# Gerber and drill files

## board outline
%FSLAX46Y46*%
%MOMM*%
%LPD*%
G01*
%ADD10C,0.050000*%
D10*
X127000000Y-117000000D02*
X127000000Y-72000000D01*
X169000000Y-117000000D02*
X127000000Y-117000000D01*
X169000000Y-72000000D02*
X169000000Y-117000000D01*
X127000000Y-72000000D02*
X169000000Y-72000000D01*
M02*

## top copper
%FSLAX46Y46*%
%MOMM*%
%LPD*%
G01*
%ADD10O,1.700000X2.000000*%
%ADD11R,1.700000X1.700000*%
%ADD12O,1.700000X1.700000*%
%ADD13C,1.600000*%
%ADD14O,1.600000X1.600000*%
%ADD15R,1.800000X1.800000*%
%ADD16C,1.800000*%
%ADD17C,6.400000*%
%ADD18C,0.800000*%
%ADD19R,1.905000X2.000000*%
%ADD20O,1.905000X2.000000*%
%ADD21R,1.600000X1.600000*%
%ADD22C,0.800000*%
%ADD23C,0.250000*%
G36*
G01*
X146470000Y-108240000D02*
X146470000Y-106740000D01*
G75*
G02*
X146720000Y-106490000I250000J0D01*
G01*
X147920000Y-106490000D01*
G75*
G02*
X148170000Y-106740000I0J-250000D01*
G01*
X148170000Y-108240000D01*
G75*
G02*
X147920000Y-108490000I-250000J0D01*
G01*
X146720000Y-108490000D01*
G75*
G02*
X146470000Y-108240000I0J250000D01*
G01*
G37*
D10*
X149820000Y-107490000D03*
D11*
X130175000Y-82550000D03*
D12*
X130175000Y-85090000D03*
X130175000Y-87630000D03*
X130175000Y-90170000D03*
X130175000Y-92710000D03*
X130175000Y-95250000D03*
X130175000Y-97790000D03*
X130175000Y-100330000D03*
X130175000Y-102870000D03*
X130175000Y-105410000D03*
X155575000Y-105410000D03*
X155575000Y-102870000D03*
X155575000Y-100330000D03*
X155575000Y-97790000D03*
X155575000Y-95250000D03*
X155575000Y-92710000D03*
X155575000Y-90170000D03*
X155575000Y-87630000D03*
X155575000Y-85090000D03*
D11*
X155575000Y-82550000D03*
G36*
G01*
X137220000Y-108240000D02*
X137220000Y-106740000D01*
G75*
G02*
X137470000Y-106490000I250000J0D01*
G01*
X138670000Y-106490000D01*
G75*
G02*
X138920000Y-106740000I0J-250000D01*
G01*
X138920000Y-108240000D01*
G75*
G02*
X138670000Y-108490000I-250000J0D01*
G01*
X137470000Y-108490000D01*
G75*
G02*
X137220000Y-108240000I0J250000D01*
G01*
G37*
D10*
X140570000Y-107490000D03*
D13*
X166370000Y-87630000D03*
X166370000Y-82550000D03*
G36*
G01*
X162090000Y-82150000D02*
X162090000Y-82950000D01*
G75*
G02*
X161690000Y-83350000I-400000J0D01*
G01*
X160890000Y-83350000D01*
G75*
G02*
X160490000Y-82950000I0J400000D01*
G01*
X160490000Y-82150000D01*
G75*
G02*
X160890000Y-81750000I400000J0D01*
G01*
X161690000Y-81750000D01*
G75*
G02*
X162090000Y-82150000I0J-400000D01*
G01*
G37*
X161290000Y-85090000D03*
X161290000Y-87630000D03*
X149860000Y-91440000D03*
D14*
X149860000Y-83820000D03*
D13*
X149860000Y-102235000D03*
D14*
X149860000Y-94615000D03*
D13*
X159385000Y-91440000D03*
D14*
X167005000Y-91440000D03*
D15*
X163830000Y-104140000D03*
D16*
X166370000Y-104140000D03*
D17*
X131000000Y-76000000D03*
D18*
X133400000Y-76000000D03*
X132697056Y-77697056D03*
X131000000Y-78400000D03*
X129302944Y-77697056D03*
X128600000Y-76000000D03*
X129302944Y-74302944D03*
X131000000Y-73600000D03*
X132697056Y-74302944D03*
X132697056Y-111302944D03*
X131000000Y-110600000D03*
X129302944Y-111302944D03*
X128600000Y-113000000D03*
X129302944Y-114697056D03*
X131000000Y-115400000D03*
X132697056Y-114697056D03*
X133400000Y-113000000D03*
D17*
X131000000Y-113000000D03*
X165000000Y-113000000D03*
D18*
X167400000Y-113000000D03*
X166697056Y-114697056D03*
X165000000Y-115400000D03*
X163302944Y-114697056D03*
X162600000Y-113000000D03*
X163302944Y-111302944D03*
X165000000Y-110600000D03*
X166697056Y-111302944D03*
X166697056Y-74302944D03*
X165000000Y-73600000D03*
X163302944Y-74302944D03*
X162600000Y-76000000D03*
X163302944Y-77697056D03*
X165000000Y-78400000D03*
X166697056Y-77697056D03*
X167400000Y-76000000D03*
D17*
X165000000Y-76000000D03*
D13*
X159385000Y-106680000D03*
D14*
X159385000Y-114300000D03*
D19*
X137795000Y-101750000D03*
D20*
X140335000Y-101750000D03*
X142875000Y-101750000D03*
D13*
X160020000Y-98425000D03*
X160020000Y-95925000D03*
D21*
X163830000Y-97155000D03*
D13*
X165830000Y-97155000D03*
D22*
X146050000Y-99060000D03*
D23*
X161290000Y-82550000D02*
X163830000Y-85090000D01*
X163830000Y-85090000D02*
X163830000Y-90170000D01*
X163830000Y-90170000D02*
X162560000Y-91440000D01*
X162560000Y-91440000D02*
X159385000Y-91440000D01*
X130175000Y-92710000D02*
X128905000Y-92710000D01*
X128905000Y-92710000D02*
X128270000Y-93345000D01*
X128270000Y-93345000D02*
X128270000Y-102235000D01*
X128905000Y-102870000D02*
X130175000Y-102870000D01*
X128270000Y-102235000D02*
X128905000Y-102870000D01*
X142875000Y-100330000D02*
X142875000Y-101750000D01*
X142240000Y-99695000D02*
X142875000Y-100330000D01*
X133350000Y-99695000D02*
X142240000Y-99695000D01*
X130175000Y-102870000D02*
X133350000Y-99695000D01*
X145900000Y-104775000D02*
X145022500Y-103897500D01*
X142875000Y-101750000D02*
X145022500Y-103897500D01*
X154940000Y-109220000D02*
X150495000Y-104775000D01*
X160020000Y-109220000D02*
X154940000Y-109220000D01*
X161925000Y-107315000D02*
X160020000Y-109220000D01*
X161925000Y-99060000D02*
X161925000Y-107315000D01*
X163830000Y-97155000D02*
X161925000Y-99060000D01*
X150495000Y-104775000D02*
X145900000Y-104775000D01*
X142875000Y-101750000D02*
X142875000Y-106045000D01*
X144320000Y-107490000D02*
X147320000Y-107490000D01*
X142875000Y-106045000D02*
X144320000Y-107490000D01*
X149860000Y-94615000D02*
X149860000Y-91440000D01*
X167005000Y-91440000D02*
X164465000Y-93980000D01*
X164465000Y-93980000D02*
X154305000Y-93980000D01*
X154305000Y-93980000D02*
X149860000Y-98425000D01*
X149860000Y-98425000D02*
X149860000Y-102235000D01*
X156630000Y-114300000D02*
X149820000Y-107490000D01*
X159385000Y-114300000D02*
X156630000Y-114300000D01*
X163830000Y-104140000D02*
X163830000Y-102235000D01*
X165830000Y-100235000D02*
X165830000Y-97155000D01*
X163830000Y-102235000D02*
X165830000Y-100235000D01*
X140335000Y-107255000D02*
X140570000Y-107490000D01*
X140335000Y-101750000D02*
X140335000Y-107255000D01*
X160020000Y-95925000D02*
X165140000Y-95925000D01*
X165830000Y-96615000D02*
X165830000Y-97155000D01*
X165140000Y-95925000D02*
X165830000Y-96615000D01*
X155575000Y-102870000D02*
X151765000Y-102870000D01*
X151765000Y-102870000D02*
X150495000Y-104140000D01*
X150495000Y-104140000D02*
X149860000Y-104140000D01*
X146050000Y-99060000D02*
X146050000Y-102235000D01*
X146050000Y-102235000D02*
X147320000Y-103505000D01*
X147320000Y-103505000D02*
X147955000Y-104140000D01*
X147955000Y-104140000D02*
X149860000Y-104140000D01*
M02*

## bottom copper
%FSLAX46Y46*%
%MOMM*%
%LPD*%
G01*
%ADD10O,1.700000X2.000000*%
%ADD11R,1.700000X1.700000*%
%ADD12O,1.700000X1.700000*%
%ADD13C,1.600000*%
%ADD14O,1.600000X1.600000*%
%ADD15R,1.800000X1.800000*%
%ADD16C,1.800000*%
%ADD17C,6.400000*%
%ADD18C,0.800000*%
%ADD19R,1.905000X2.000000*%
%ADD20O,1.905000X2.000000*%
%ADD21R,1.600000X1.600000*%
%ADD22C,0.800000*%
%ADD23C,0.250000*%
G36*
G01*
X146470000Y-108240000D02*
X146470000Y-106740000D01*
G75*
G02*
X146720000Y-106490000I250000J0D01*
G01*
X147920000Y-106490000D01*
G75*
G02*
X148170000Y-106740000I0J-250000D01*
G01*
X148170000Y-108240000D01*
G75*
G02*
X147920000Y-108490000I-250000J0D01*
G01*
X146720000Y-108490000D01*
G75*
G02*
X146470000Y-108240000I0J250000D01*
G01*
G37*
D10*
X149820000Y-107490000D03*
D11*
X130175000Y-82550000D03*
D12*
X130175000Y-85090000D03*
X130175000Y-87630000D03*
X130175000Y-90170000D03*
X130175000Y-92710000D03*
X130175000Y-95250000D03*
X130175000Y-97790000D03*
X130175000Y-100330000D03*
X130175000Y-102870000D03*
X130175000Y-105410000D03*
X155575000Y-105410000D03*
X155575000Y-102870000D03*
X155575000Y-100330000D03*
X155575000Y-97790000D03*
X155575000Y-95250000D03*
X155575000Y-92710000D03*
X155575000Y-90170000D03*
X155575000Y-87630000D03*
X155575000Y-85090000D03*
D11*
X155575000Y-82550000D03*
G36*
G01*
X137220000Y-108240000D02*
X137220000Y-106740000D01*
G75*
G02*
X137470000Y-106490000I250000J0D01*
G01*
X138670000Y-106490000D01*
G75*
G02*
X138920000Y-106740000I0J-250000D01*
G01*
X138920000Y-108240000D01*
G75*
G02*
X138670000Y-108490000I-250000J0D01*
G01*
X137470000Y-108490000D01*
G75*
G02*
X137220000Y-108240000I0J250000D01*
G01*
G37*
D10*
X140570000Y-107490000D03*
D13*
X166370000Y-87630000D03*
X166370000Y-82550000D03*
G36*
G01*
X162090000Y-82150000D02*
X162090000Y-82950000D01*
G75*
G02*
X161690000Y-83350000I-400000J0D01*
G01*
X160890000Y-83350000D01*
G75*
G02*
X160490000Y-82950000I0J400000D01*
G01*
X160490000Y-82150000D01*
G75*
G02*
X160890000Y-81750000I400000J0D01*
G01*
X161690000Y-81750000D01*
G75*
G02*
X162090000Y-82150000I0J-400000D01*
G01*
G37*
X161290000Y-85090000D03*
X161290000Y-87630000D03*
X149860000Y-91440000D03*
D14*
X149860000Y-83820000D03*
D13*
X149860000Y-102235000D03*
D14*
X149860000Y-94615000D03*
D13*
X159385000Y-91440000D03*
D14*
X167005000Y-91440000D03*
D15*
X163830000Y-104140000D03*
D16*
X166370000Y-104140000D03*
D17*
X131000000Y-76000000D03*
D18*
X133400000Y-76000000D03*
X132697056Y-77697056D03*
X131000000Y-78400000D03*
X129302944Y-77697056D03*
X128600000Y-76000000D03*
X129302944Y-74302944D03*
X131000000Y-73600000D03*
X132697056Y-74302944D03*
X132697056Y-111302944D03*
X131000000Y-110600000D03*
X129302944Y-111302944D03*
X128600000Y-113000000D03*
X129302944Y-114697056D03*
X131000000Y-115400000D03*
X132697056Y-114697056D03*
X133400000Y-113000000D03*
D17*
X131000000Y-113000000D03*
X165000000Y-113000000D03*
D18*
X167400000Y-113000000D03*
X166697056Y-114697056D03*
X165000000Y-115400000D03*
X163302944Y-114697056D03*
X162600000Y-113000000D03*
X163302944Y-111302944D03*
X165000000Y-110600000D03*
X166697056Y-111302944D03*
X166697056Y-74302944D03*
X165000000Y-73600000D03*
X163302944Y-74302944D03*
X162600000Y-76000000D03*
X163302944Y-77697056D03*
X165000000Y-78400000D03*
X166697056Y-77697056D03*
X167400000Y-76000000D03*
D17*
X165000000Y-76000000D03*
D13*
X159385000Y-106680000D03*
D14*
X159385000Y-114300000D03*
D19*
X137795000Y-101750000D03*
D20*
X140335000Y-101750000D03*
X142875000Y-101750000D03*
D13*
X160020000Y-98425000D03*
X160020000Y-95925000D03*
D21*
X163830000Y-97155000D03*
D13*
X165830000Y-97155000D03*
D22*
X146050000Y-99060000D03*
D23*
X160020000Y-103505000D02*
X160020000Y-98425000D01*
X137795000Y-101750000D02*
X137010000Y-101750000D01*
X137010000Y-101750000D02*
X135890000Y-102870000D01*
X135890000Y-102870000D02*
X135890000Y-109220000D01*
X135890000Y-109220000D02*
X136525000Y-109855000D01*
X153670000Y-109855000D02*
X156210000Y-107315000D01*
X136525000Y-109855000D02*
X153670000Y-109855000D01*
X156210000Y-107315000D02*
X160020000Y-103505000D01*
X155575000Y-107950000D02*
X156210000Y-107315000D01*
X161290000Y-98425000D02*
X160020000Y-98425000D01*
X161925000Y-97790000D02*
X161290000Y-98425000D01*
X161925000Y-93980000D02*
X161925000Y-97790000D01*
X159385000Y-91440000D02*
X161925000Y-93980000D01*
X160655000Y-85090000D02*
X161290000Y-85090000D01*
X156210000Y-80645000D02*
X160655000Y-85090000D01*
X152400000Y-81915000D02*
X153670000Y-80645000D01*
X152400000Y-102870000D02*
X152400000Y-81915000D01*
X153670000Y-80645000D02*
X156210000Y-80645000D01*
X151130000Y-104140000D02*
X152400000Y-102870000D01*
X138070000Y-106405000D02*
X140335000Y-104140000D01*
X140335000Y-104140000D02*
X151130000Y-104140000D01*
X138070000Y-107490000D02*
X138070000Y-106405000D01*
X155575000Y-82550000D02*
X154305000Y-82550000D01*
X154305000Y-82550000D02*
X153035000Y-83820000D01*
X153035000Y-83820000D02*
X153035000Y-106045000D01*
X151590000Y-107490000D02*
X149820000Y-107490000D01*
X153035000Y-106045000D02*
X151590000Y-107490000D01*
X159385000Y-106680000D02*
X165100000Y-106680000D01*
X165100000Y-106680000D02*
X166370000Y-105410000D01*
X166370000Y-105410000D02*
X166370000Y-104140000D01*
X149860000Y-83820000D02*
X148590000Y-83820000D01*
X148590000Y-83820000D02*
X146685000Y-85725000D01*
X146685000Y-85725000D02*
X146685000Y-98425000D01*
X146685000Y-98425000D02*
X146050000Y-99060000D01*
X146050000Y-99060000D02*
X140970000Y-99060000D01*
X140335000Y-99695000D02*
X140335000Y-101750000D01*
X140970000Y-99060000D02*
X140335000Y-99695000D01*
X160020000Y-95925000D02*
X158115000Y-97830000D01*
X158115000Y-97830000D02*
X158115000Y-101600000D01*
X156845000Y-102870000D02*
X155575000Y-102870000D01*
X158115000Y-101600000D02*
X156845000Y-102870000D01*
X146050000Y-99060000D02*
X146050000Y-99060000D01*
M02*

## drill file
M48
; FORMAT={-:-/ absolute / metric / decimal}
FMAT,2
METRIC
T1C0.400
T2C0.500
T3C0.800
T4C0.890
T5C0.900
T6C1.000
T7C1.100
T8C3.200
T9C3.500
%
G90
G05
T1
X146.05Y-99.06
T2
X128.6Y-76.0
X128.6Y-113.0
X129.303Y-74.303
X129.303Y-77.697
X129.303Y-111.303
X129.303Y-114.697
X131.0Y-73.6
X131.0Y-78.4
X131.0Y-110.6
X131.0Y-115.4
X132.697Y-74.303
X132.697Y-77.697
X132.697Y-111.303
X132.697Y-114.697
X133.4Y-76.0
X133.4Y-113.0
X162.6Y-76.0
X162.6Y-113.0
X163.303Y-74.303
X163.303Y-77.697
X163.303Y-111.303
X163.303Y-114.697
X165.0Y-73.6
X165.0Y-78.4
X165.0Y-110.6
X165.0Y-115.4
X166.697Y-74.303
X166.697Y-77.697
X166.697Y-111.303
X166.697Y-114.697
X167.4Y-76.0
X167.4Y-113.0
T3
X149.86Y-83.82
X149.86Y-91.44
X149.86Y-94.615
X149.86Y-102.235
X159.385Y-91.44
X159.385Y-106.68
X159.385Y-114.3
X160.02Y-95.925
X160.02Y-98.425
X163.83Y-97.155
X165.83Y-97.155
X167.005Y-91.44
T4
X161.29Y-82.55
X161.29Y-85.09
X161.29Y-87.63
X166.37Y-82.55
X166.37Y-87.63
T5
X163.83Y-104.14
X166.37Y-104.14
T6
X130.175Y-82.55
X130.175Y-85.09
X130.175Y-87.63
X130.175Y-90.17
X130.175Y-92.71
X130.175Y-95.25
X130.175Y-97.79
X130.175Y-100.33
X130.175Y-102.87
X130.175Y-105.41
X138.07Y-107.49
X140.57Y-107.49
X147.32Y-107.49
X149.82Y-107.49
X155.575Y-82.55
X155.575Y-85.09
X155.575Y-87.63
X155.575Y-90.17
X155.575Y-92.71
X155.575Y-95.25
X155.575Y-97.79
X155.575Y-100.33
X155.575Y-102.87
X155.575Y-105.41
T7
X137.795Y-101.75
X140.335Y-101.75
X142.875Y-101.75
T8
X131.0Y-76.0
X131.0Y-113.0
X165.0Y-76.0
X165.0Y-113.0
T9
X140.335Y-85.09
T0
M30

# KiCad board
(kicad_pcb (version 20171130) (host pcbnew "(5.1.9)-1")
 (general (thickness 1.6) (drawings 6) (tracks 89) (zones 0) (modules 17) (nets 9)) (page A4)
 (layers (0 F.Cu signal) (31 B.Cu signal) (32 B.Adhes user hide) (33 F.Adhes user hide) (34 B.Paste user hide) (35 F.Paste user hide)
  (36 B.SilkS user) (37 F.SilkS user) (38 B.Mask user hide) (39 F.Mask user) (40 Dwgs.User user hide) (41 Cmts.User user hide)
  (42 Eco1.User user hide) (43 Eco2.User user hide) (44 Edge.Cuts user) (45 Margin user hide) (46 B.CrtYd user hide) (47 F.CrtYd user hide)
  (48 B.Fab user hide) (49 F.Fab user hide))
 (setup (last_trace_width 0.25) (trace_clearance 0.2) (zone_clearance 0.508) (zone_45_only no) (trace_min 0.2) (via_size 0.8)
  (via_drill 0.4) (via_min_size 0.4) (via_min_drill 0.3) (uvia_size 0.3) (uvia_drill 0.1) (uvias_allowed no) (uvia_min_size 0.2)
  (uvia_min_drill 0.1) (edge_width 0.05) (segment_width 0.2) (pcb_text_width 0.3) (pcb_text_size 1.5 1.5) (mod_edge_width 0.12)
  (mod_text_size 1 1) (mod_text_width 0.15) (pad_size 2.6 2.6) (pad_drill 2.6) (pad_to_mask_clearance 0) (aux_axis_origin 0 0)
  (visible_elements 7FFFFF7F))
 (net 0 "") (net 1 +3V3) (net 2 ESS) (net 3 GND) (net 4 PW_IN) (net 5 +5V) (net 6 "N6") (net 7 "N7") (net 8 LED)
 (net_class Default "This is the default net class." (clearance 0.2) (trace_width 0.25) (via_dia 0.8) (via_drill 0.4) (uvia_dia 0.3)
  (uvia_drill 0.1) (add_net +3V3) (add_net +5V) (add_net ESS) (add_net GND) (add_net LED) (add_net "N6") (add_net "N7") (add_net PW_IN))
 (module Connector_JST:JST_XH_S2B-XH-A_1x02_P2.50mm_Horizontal (layer F.Cu) (at 147.32 107.49)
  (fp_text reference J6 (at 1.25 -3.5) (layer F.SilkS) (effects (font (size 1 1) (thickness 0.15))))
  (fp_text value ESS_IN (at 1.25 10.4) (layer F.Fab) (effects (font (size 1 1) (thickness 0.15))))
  (pad 1 thru_hole roundrect (at 0 0) (size 1.7 2) (drill 1) (layers *.Cu *.Mask) (roundrect_rratio 0.1470588235294118) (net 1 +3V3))
  (pad 2 thru_hole oval (at 2.5 0) (size 1.7 2) (drill 1) (layers *.Cu *.Mask) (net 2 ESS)))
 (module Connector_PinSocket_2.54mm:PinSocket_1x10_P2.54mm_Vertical (layer F.Cu) (at 130.175 82.55)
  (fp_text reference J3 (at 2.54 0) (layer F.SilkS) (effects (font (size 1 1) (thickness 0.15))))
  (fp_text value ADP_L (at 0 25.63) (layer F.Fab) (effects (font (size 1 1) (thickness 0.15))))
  (pad 1 thru_hole rect (at 0 0) (size 1.7 1.7) (drill 1) (layers *.Cu *.Mask))
  (pad 2 thru_hole oval (at 0 2.54) (size 1.7 1.7) (drill 1) (layers *.Cu *.Mask))
  (pad 3 thru_hole oval (at 0 5.08) (size 1.7 1.7) (drill 1) (layers *.Cu *.Mask))
  (pad 4 thru_hole oval (at 0 7.62) (size 1.7 1.7) (drill 1) (layers *.Cu *.Mask))
  (pad 5 thru_hole oval (at 0 10.16) (size 1.7 1.7) (drill 1) (layers *.Cu *.Mask) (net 1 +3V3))
  (pad 6 thru_hole oval (at 0 12.7) (size 1.7 1.7) (drill 1) (layers *.Cu *.Mask))
  (pad 7 thru_hole oval (at 0 15.24) (size 1.7 1.7) (drill 1) (layers *.Cu *.Mask))
  (pad 8 thru_hole oval (at 0 17.78) (size 1.7 1.7) (drill 1) (layers *.Cu *.Mask))
  (pad 9 thru_hole oval (at 0 20.32) (size 1.7 1.7) (drill 1) (layers *.Cu *.Mask) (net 1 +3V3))
  (pad 10 thru_hole oval (at 0 22.86) (size 1.7 1.7) (drill 1) (layers *.Cu *.Mask)))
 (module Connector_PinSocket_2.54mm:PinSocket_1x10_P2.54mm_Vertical (layer F.Cu) (at 155.575 82.55)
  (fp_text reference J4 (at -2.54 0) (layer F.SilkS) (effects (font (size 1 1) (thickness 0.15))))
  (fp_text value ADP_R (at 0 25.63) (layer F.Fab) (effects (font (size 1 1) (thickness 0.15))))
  (pad 10 thru_hole oval (at 0 22.86) (size 1.7 1.7) (drill 1) (layers *.Cu *.Mask))
  (pad 9 thru_hole oval (at 0 20.32) (size 1.7 1.7) (drill 1) (layers *.Cu *.Mask) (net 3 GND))
  (pad 8 thru_hole oval (at 0 17.78) (size 1.7 1.7) (drill 1) (layers *.Cu *.Mask))
  (pad 7 thru_hole oval (at 0 15.24) (size 1.7 1.7) (drill 1) (layers *.Cu *.Mask))
  (pad 6 thru_hole oval (at 0 12.7) (size 1.7 1.7) (drill 1) (layers *.Cu *.Mask))
  (pad 5 thru_hole oval (at 0 10.16) (size 1.7 1.7) (drill 1) (layers *.Cu *.Mask))
  (pad 4 thru_hole oval (at 0 7.62) (size 1.7 1.7) (drill 1) (layers *.Cu *.Mask))
  (pad 3 thru_hole oval (at 0 5.08) (size 1.7 1.7) (drill 1) (layers *.Cu *.Mask))
  (pad 2 thru_hole oval (at 0 2.54) (size 1.7 1.7) (drill 1) (layers *.Cu *.Mask))
  (pad 1 thru_hole rect (at 0 0) (size 1.7 1.7) (drill 1) (layers *.Cu *.Mask) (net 2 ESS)))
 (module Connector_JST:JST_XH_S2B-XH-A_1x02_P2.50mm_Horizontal (layer F.Cu) (at 138.07 107.49)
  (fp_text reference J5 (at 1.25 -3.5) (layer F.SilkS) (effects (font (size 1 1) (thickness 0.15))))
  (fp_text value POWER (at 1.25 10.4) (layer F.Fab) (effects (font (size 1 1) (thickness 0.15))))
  (pad 1 thru_hole roundrect (at 0 0) (size 1.7 2) (drill 1) (layers *.Cu *.Mask) (roundrect_rratio 0.1470588235294118) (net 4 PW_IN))
  (pad 2 thru_hole oval (at 2.5 0) (size 1.7 2) (drill 1) (layers *.Cu *.Mask) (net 3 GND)))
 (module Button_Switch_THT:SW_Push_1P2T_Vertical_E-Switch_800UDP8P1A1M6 (layer F.Cu) (at 161.29 82.55)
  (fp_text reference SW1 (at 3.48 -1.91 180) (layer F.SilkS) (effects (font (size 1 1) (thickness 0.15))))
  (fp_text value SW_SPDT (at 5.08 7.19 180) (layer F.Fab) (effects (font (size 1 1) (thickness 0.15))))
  (pad "" thru_hole circle (at 5.08 5.08 180) (size 1.6 1.6) (drill 0.89) (layers *.Cu *.Mask))
  (pad "" thru_hole circle (at 5.08 0 180) (size 1.6 1.6) (drill 0.89) (layers *.Cu *.Mask))
  (pad 1 thru_hole roundrect (at 0 0 180) (size 1.6 1.6) (drill 0.89) (layers *.Cu *.Mask) (roundrect_rratio 0.25) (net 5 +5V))
  (pad 2 thru_hole circle (at 0 2.54 180) (size 1.6 1.6) (drill 0.89) (layers *.Cu *.Mask) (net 4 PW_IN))
  (pad 3 thru_hole circle (at 0 5.08 180) (size 1.6 1.6) (drill 0.89) (layers *.Cu *.Mask)))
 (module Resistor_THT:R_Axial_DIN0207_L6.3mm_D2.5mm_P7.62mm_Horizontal (layer F.Cu) (at 149.86 91.44 90)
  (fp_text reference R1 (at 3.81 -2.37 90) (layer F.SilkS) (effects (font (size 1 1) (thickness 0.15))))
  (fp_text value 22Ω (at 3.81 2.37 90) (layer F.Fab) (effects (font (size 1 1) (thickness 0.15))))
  (pad 1 thru_hole circle (at 0 0 90) (size 1.6 1.6) (drill 0.8) (layers *.Cu *.Mask) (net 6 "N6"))
  (pad 2 thru_hole oval (at 7.62 0 90) (size 1.6 1.6) (drill 0.8) (layers *.Cu *.Mask) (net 3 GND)))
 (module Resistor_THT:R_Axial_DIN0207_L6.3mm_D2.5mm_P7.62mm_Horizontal (layer F.Cu) (at 149.86 102.235 90)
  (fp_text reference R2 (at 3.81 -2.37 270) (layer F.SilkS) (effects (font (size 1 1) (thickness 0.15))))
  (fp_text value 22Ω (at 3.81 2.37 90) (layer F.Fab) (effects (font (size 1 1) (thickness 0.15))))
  (pad 1 thru_hole circle (at 0 0 90) (size 1.6 1.6) (drill 0.8) (layers *.Cu *.Mask) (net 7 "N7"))
  (pad 2 thru_hole oval (at 7.62 0 90) (size 1.6 1.6) (drill 0.8) (layers *.Cu *.Mask) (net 6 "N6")))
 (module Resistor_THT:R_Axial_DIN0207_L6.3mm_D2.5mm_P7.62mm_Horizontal (layer F.Cu) (at 159.385 91.44)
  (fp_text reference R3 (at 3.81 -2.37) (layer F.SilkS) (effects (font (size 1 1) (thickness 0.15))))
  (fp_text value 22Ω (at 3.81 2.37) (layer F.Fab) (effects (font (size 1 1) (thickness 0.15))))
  (pad 1 thru_hole circle (at 0 0) (size 1.6 1.6) (drill 0.8) (layers *.Cu *.Mask) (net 5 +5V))
  (pad 2 thru_hole oval (at 7.62 0) (size 1.6 1.6) (drill 0.8) (layers *.Cu *.Mask) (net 7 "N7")))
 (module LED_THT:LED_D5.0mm (layer F.Cu) (at 163.83 104.14)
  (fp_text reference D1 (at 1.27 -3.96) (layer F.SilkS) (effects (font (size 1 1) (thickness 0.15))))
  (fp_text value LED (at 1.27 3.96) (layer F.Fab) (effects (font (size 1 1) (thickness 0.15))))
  (pad 1 thru_hole rect (at 0 0) (size 1.8 1.8) (drill 0.9) (layers *.Cu *.Mask) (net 3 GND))
  (pad 2 thru_hole circle (at 2.54 0) (size 1.8 1.8) (drill 0.9) (layers *.Cu *.Mask) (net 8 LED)))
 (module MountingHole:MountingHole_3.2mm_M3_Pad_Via (layer F.Cu) (at 131 76)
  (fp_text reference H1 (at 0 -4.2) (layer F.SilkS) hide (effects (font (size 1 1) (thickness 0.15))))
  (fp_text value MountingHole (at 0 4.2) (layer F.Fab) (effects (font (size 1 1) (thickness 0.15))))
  (pad 1 thru_hole circle (at 0 0) (size 6.4 6.4) (drill 3.2) (layers *.Cu *.Mask))
  (pad 1 thru_hole circle (at 2.4 0) (size 0.8 0.8) (drill 0.5) (layers *.Cu *.Mask))
  (pad 1 thru_hole circle (at 1.697056 1.697056) (size 0.8 0.8) (drill 0.5) (layers *.Cu *.Mask))
  (pad 1 thru_hole circle (at 0 2.4) (size 0.8 0.8) (drill 0.5) (layers *.Cu *.Mask))
  (pad 1 thru_hole circle (at -1.697056 1.697056) (size 0.8 0.8) (drill 0.5) (layers *.Cu *.Mask))
  (pad 1 thru_hole circle (at -2.4 0) (size 0.8 0.8) (drill 0.5) (layers *.Cu *.Mask))
  (pad 1 thru_hole circle (at -1.697056 -1.697056) (size 0.8 0.8) (drill 0.5) (layers *.Cu *.Mask))
  (pad 1 thru_hole circle (at 0 -2.4) (size 0.8 0.8) (drill 0.5) (layers *.Cu *.Mask))
  (pad 1 thru_hole circle (at 1.697056 -1.697056) (size 0.8 0.8) (drill 0.5) (layers *.Cu *.Mask)))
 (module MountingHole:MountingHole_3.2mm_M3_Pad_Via (layer F.Cu) (at 131 113)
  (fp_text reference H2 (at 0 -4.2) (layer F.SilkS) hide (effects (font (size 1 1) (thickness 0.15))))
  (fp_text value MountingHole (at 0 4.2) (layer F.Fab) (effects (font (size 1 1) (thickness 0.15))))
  (pad 1 thru_hole circle (at 1.697056 -1.697056) (size 0.8 0.8) (drill 0.5) (layers *.Cu *.Mask))
  (pad 1 thru_hole circle (at 0 -2.4) (size 0.8 0.8) (drill 0.5) (layers *.Cu *.Mask))
  (pad 1 thru_hole circle (at -1.697056 -1.697056) (size 0.8 0.8) (drill 0.5) (layers *.Cu *.Mask))
  (pad 1 thru_hole circle (at -2.4 0) (size 0.8 0.8) (drill 0.5) (layers *.Cu *.Mask))
  (pad 1 thru_hole circle (at -1.697056 1.697056) (size 0.8 0.8) (drill 0.5) (layers *.Cu *.Mask))
  (pad 1 thru_hole circle (at 0 2.4) (size 0.8 0.8) (drill 0.5) (layers *.Cu *.Mask))
  (pad 1 thru_hole circle (at 1.697056 1.697056) (size 0.8 0.8) (drill 0.5) (layers *.Cu *.Mask))
  (pad 1 thru_hole circle (at 2.4 0) (size 0.8 0.8) (drill 0.5) (layers *.Cu *.Mask))
  (pad 1 thru_hole circle (at 0 0) (size 6.4 6.4) (drill 3.2) (layers *.Cu *.Mask)))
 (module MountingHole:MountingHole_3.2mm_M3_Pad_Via (layer F.Cu) (at 165 113)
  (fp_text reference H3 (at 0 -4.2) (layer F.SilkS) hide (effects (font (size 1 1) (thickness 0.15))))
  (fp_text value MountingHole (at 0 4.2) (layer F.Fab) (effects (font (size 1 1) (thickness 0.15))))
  (pad 1 thru_hole circle (at 0 0) (size 6.4 6.4) (drill 3.2) (layers *.Cu *.Mask))
  (pad 1 thru_hole circle (at 2.4 0) (size 0.8 0.8) (drill 0.5) (layers *.Cu *.Mask))
  (pad 1 thru_hole circle (at 1.697056 1.697056) (size 0.8 0.8) (drill 0.5) (layers *.Cu *.Mask))
  (pad 1 thru_hole circle (at 0 2.4) (size 0.8 0.8) (drill 0.5) (layers *.Cu *.Mask))
  (pad 1 thru_hole circle (at -1.697056 1.697056) (size 0.8 0.8) (drill 0.5) (layers *.Cu *.Mask))
  (pad 1 thru_hole circle (at -2.4 0) (size 0.8 0.8) (drill 0.5) (layers *.Cu *.Mask))
  (pad 1 thru_hole circle (at -1.697056 -1.697056) (size 0.8 0.8) (drill 0.5) (layers *.Cu *.Mask))
  (pad 1 thru_hole circle (at 0 -2.4) (size 0.8 0.8) (drill 0.5) (layers *.Cu *.Mask))
  (pad 1 thru_hole circle (at 1.697056 -1.697056) (size 0.8 0.8) (drill 0.5) (layers *.Cu *.Mask)))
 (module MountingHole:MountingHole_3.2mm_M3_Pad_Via (layer F.Cu) (at 165 76)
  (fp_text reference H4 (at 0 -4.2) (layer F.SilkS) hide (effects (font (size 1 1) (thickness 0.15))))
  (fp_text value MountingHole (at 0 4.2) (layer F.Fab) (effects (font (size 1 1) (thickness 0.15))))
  (pad 1 thru_hole circle (at 1.697056 -1.697056) (size 0.8 0.8) (drill 0.5) (layers *.Cu *.Mask))
  (pad 1 thru_hole circle (at 0 -2.4) (size 0.8 0.8) (drill 0.5) (layers *.Cu *.Mask))
  (pad 1 thru_hole circle (at -1.697056 -1.697056) (size 0.8 0.8) (drill 0.5) (layers *.Cu *.Mask))
  (pad 1 thru_hole circle (at -2.4 0) (size 0.8 0.8) (drill 0.5) (layers *.Cu *.Mask))
  (pad 1 thru_hole circle (at -1.697056 1.697056) (size 0.8 0.8) (drill 0.5) (layers *.Cu *.Mask))
  (pad 1 thru_hole circle (at 0 2.4) (size 0.8 0.8) (drill 0.5) (layers *.Cu *.Mask))
  (pad 1 thru_hole circle (at 1.697056 1.697056) (size 0.8 0.8) (drill 0.5) (layers *.Cu *.Mask))
  (pad 1 thru_hole circle (at 2.4 0) (size 0.8 0.8) (drill 0.5) (layers *.Cu *.Mask))
  (pad 1 thru_hole circle (at 0 0) (size 6.4 6.4) (drill 3.2) (layers *.Cu *.Mask)))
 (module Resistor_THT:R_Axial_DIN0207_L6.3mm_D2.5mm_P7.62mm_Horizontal (layer F.Cu) (at 159.385 106.68 270)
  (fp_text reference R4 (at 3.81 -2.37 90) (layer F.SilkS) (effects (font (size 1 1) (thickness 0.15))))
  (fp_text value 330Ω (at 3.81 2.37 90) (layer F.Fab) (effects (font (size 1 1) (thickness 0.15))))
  (pad 1 thru_hole circle (at 0 0 270) (size 1.6 1.6) (drill 0.8) (layers *.Cu *.Mask) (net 8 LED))
  (pad 2 thru_hole oval (at 7.62 0 270) (size 1.6 1.6) (drill 0.8) (layers *.Cu *.Mask) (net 2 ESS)))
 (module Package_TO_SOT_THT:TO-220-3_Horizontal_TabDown (layer F.Cu) (at 137.795 101.75)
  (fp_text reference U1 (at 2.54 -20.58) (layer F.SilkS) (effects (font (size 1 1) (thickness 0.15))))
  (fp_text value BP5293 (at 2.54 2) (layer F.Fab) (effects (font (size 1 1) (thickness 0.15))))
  (pad "" np_thru_hole oval (at 2.54 -16.66) (size 3.5 3.5) (drill 3.5) (layers *.Cu *.Mask))
  (pad 1 thru_hole rect (at 0 0) (size 1.905 2) (drill 1.1) (layers *.Cu *.Mask) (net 5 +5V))
  (pad 2 thru_hole oval (at 2.54 0) (size 1.905 2) (drill 1.1) (layers *.Cu *.Mask) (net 3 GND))
  (pad 3 thru_hole oval (at 5.08 0) (size 1.905 2) (drill 1.1) (layers *.Cu *.Mask) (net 1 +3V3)))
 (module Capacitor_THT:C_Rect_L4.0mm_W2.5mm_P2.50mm (layer F.Cu) (at 160.02 98.425 90)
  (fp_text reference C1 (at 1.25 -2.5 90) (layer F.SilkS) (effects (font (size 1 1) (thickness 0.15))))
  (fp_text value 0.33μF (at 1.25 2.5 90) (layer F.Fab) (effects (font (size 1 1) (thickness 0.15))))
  (pad 1 thru_hole circle (at 0 0 90) (size 1.6 1.6) (drill 0.8) (layers *.Cu *.Mask) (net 5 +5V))
  (pad 2 thru_hole circle (at 2.5 0 90) (size 1.6 1.6) (drill 0.8) (layers *.Cu *.Mask) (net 3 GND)))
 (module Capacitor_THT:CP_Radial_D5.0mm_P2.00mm (layer F.Cu) (at 163.83 97.155)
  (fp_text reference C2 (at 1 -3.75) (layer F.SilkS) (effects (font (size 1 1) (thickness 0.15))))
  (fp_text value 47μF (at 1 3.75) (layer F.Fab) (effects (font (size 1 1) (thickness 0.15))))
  (pad 1 thru_hole rect (at 0 0) (size 1.6 1.6) (drill 0.8) (layers *.Cu *.Mask) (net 1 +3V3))
  (pad 2 thru_hole circle (at 2 0) (size 1.6 1.6) (drill 0.8) (layers *.Cu *.Mask) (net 3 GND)))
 (gr_line (start 127 117) (end 127 72) (layer Edge.Cuts) (width 0.05))
 (gr_line (start 169 117) (end 127 117) (layer Edge.Cuts) (width 0.05))
 (gr_line (start 169 72) (end 169 117) (layer Edge.Cuts) (width 0.05))
 (gr_line (start 127 72) (end 169 72) (layer Edge.Cuts) (width 0.05))
 (segment (start 161.29 82.55) (end 163.83 85.09) (width 0.25) (layer F.Cu) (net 5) (status 10))
 (segment (start 163.83 85.09) (end 163.83 90.17) (width 0.25) (layer F.Cu) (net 5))
 (segment (start 163.83 90.17) (end 162.56 91.44) (width 0.25) (layer F.Cu) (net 5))
 (segment (start 162.56 91.44) (end 159.385 91.44) (width 0.25) (layer F.Cu) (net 5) (status 20))
 (segment (start 160.02 103.505) (end 160.02 98.425) (width 0.25) (layer B.Cu) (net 5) (status 20))
 (segment (start 137.795 101.75) (end 137.01 101.75) (width 0.25) (layer B.Cu) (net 5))
 (segment (start 137.01 101.75) (end 135.89 102.87) (width 0.25) (layer B.Cu) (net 5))
 (segment (start 135.89 102.87) (end 135.89 109.22) (width 0.25) (layer B.Cu) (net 5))
 (segment (start 135.89 109.22) (end 136.525 109.855) (width 0.25) (layer B.Cu) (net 5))
 (segment (start 153.67 109.855) (end 156.21 107.315) (width 0.25) (layer B.Cu) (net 5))
 (segment (start 136.525 109.855) (end 153.67 109.855) (width 0.25) (layer B.Cu) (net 5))
 (segment (start 156.21 107.315) (end 160.02 103.505) (width 0.25) (layer B.Cu) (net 5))
 (segment (start 155.575 107.95) (end 156.21 107.315) (width 0.25) (layer B.Cu) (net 5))
 (segment (start 161.29 98.425) (end 160.02 98.425) (width 0.25) (layer B.Cu) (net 5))
 (segment (start 161.925 97.79) (end 161.29 98.425) (width 0.25) (layer B.Cu) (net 5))
 (segment (start 161.925 93.98) (end 161.925 97.79) (width 0.25) (layer B.Cu) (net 5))
 (segment (start 159.385 91.44) (end 161.925 93.98) (width 0.25) (layer B.Cu) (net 5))
 (segment (start 130.175 92.71) (end 128.905 92.71) (width 0.25) (layer F.Cu) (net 1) (status 10))
 (segment (start 128.905 92.71) (end 128.27 93.345) (width 0.25) (layer F.Cu) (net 1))
 (segment (start 128.27 93.345) (end 128.27 102.235) (width 0.25) (layer F.Cu) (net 1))
 (segment (start 128.905 102.87) (end 130.175 102.87) (width 0.25) (layer F.Cu) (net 1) (status 20))
 (segment (start 128.27 102.235) (end 128.905 102.87) (width 0.25) (layer F.Cu) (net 1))
 (segment (start 142.875 100.33) (end 142.875 101.75) (width 0.25) (layer F.Cu) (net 1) (status 20))
 (segment (start 142.24 99.695) (end 142.875 100.33) (width 0.25) (layer F.Cu) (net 1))
 (segment (start 133.35 99.695) (end 142.24 99.695) (width 0.25) (layer F.Cu) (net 1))
 (segment (start 130.175 102.87) (end 133.35 99.695) (width 0.25) (layer F.Cu) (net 1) (status 10))
 (segment (start 145.9 104.775) (end 145.0225 103.8975) (width 0.25) (layer F.Cu) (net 1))
 (segment (start 142.875 101.75) (end 145.0225 103.8975) (width 0.25) (layer F.Cu) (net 1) (status 10))
 (segment (start 154.94 109.22) (end 150.495 104.775) (width 0.25) (layer F.Cu) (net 1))
 (segment (start 160.02 109.22) (end 154.94 109.22) (width 0.25) (layer F.Cu) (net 1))
 (segment (start 161.925 107.315) (end 160.02 109.22) (width 0.25) (layer F.Cu) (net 1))
 (segment (start 161.925 99.06) (end 161.925 107.315) (width 0.25) (layer F.Cu) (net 1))
 (segment (start 163.83 97.155) (end 161.925 99.06) (width 0.25) (layer F.Cu) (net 1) (status 10))
 (segment (start 150.495 104.775) (end 145.9 104.775) (width 0.25) (layer F.Cu) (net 1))
 (segment (start 142.875 101.75) (end 142.875 106.045) (width 0.25) (layer F.Cu) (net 1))
 (segment (start 144.32 107.49) (end 147.32 107.49) (width 0.25) (layer F.Cu) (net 1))
 (segment (start 142.875 106.045) (end 144.32 107.49) (width 0.25) (layer F.Cu) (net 1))
 (segment (start 160.655 85.09) (end 161.29 85.09) (width 0.25) (layer B.Cu) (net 4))
 (segment (start 156.21 80.645) (end 160.655 85.09) (width 0.25) (layer B.Cu) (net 4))
 (segment (start 152.4 81.915) (end 153.67 80.645) (width 0.25) (layer B.Cu) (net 4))
 (segment (start 152.4 102.87) (end 152.4 81.915) (width 0.25) (layer B.Cu) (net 4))
 (segment (start 153.67 80.645) (end 156.21 80.645) (width 0.25) (layer B.Cu) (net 4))
 (segment (start 151.13 104.14) (end 152.4 102.87) (width 0.25) (layer B.Cu) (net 4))
 (segment (start 138.07 106.405) (end 140.335 104.14) (width 0.25) (layer B.Cu) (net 4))
 (segment (start 140.335 104.14) (end 151.13 104.14) (width 0.25) (layer B.Cu) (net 4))
 (segment (start 138.07 107.49) (end 138.07 106.405) (width 0.25) (layer B.Cu) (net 4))
 (segment (start 149.86 94.615) (end 149.86 91.44) (width 0.25) (layer F.Cu) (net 6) (status 30))
 (segment (start 167.005 91.44) (end 164.465 93.98) (width 0.25) (layer F.Cu) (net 7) (status 10))
 (segment (start 164.465 93.98) (end 154.305 93.98) (width 0.25) (layer F.Cu) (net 7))
 (segment (start 154.305 93.98) (end 149.86 98.425) (width 0.25) (layer F.Cu) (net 7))
 (segment (start 149.86 98.425) (end 149.86 102.235) (width 0.25) (layer F.Cu) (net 7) (status 20))
 (segment (start 156.63 114.3) (end 149.82 107.49) (width 0.25) (layer F.Cu) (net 2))
 (segment (start 159.385 114.3) (end 156.63 114.3) (width 0.25) (layer F.Cu) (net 2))
 (segment (start 155.575 82.55) (end 154.305 82.55) (width 0.25) (layer B.Cu) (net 2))
 (segment (start 154.305 82.55) (end 153.035 83.82) (width 0.25) (layer B.Cu) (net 2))
 (segment (start 153.035 83.82) (end 153.035 106.045) (width 0.25) (layer B.Cu) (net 2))
 (segment (start 151.59 107.49) (end 149.82 107.49) (width 0.25) (layer B.Cu) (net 2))
 (segment (start 153.035 106.045) (end 151.59 107.49) (width 0.25) (layer B.Cu) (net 2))
 (segment (start 159.385 106.68) (end 165.1 106.68) (width 0.25) (layer B.Cu) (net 8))
 (segment (start 165.1 106.68) (end 166.37 105.41) (width 0.25) (layer B.Cu) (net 8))
 (segment (start 166.37 105.41) (end 166.37 104.14) (width 0.25) (layer B.Cu) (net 8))
 (segment (start 163.83 104.14) (end 163.83 102.235) (width 0.25) (layer F.Cu) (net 3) (status 10))
 (segment (start 165.83 100.235) (end 165.83 97.155) (width 0.25) (layer F.Cu) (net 3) (status 20))
 (segment (start 163.83 102.235) (end 165.83 100.235) (width 0.25) (layer F.Cu) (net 3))
 (segment (start 140.335 107.255) (end 140.57 107.49) (width 0.25) (layer F.Cu) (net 3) (status 30))
 (segment (start 140.335 101.75) (end 140.335 107.255) (width 0.25) (layer F.Cu) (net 3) (status 30))
 (segment (start 149.86 83.82) (end 148.59 83.82) (width 0.25) (layer B.Cu) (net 3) (status 10))
 (segment (start 148.59 83.82) (end 146.685 85.725) (width 0.25) (layer B.Cu) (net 3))
 (segment (start 146.685 85.725) (end 146.685 98.425) (width 0.25) (layer B.Cu) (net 3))
 (segment (start 146.685 98.425) (end 146.05 99.06) (width 0.25) (layer B.Cu) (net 3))
 (segment (start 146.05 99.06) (end 140.97 99.06) (width 0.25) (layer B.Cu) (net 3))
 (segment (start 140.335 99.695) (end 140.335 101.75) (width 0.25) (layer B.Cu) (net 3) (status 20))
 (segment (start 140.97 99.06) (end 140.335 99.695) (width 0.25) (layer B.Cu) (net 3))
 (segment (start 160.02 95.925) (end 165.14 95.925) (width 0.25) (layer F.Cu) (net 3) (status 10))
 (segment (start 165.83 96.615) (end 165.83 97.155) (width 0.25) (layer F.Cu) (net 3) (status 30))
 (segment (start 165.14 95.925) (end 165.83 96.615) (width 0.25) (layer F.Cu) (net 3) (status 20))
 (segment (start 160.02 95.925) (end 158.115 97.83) (width 0.25) (layer B.Cu) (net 3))
 (segment (start 158.115 97.83) (end 158.115 101.6) (width 0.25) (layer B.Cu) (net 3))
 (segment (start 156.845 102.87) (end 155.575 102.87) (width 0.25) (layer B.Cu) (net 3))
 (segment (start 158.115 101.6) (end 156.845 102.87) (width 0.25) (layer B.Cu) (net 3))
 (segment (start 155.575 102.87) (end 151.765 102.87) (width 0.25) (layer F.Cu) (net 3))
 (segment (start 151.765 102.87) (end 150.495 104.14) (width 0.25) (layer F.Cu) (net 3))
 (segment (start 150.495 104.14) (end 149.86 104.14) (width 0.25) (layer F.Cu) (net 3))
 (segment (start 146.05 99.06) (end 146.05 99.06) (width 0.25) (layer B.Cu) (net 3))
 (via (at 146.05 99.06) (size 0.8) (drill 0.4) (layers F.Cu B.Cu) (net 3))
 (segment (start 146.05 99.06) (end 146.05 102.235) (width 0.25) (layer F.Cu) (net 3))
 (segment (start 146.05 102.235) (end 147.32 103.505) (width 0.25) (layer F.Cu) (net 3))
 (segment (start 147.32 103.505) (end 147.955 104.14) (width 0.25) (layer F.Cu) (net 3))
 (segment (start 147.955 104.14) (end 149.86 104.14) (width 0.25) (layer F.Cu) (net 3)))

